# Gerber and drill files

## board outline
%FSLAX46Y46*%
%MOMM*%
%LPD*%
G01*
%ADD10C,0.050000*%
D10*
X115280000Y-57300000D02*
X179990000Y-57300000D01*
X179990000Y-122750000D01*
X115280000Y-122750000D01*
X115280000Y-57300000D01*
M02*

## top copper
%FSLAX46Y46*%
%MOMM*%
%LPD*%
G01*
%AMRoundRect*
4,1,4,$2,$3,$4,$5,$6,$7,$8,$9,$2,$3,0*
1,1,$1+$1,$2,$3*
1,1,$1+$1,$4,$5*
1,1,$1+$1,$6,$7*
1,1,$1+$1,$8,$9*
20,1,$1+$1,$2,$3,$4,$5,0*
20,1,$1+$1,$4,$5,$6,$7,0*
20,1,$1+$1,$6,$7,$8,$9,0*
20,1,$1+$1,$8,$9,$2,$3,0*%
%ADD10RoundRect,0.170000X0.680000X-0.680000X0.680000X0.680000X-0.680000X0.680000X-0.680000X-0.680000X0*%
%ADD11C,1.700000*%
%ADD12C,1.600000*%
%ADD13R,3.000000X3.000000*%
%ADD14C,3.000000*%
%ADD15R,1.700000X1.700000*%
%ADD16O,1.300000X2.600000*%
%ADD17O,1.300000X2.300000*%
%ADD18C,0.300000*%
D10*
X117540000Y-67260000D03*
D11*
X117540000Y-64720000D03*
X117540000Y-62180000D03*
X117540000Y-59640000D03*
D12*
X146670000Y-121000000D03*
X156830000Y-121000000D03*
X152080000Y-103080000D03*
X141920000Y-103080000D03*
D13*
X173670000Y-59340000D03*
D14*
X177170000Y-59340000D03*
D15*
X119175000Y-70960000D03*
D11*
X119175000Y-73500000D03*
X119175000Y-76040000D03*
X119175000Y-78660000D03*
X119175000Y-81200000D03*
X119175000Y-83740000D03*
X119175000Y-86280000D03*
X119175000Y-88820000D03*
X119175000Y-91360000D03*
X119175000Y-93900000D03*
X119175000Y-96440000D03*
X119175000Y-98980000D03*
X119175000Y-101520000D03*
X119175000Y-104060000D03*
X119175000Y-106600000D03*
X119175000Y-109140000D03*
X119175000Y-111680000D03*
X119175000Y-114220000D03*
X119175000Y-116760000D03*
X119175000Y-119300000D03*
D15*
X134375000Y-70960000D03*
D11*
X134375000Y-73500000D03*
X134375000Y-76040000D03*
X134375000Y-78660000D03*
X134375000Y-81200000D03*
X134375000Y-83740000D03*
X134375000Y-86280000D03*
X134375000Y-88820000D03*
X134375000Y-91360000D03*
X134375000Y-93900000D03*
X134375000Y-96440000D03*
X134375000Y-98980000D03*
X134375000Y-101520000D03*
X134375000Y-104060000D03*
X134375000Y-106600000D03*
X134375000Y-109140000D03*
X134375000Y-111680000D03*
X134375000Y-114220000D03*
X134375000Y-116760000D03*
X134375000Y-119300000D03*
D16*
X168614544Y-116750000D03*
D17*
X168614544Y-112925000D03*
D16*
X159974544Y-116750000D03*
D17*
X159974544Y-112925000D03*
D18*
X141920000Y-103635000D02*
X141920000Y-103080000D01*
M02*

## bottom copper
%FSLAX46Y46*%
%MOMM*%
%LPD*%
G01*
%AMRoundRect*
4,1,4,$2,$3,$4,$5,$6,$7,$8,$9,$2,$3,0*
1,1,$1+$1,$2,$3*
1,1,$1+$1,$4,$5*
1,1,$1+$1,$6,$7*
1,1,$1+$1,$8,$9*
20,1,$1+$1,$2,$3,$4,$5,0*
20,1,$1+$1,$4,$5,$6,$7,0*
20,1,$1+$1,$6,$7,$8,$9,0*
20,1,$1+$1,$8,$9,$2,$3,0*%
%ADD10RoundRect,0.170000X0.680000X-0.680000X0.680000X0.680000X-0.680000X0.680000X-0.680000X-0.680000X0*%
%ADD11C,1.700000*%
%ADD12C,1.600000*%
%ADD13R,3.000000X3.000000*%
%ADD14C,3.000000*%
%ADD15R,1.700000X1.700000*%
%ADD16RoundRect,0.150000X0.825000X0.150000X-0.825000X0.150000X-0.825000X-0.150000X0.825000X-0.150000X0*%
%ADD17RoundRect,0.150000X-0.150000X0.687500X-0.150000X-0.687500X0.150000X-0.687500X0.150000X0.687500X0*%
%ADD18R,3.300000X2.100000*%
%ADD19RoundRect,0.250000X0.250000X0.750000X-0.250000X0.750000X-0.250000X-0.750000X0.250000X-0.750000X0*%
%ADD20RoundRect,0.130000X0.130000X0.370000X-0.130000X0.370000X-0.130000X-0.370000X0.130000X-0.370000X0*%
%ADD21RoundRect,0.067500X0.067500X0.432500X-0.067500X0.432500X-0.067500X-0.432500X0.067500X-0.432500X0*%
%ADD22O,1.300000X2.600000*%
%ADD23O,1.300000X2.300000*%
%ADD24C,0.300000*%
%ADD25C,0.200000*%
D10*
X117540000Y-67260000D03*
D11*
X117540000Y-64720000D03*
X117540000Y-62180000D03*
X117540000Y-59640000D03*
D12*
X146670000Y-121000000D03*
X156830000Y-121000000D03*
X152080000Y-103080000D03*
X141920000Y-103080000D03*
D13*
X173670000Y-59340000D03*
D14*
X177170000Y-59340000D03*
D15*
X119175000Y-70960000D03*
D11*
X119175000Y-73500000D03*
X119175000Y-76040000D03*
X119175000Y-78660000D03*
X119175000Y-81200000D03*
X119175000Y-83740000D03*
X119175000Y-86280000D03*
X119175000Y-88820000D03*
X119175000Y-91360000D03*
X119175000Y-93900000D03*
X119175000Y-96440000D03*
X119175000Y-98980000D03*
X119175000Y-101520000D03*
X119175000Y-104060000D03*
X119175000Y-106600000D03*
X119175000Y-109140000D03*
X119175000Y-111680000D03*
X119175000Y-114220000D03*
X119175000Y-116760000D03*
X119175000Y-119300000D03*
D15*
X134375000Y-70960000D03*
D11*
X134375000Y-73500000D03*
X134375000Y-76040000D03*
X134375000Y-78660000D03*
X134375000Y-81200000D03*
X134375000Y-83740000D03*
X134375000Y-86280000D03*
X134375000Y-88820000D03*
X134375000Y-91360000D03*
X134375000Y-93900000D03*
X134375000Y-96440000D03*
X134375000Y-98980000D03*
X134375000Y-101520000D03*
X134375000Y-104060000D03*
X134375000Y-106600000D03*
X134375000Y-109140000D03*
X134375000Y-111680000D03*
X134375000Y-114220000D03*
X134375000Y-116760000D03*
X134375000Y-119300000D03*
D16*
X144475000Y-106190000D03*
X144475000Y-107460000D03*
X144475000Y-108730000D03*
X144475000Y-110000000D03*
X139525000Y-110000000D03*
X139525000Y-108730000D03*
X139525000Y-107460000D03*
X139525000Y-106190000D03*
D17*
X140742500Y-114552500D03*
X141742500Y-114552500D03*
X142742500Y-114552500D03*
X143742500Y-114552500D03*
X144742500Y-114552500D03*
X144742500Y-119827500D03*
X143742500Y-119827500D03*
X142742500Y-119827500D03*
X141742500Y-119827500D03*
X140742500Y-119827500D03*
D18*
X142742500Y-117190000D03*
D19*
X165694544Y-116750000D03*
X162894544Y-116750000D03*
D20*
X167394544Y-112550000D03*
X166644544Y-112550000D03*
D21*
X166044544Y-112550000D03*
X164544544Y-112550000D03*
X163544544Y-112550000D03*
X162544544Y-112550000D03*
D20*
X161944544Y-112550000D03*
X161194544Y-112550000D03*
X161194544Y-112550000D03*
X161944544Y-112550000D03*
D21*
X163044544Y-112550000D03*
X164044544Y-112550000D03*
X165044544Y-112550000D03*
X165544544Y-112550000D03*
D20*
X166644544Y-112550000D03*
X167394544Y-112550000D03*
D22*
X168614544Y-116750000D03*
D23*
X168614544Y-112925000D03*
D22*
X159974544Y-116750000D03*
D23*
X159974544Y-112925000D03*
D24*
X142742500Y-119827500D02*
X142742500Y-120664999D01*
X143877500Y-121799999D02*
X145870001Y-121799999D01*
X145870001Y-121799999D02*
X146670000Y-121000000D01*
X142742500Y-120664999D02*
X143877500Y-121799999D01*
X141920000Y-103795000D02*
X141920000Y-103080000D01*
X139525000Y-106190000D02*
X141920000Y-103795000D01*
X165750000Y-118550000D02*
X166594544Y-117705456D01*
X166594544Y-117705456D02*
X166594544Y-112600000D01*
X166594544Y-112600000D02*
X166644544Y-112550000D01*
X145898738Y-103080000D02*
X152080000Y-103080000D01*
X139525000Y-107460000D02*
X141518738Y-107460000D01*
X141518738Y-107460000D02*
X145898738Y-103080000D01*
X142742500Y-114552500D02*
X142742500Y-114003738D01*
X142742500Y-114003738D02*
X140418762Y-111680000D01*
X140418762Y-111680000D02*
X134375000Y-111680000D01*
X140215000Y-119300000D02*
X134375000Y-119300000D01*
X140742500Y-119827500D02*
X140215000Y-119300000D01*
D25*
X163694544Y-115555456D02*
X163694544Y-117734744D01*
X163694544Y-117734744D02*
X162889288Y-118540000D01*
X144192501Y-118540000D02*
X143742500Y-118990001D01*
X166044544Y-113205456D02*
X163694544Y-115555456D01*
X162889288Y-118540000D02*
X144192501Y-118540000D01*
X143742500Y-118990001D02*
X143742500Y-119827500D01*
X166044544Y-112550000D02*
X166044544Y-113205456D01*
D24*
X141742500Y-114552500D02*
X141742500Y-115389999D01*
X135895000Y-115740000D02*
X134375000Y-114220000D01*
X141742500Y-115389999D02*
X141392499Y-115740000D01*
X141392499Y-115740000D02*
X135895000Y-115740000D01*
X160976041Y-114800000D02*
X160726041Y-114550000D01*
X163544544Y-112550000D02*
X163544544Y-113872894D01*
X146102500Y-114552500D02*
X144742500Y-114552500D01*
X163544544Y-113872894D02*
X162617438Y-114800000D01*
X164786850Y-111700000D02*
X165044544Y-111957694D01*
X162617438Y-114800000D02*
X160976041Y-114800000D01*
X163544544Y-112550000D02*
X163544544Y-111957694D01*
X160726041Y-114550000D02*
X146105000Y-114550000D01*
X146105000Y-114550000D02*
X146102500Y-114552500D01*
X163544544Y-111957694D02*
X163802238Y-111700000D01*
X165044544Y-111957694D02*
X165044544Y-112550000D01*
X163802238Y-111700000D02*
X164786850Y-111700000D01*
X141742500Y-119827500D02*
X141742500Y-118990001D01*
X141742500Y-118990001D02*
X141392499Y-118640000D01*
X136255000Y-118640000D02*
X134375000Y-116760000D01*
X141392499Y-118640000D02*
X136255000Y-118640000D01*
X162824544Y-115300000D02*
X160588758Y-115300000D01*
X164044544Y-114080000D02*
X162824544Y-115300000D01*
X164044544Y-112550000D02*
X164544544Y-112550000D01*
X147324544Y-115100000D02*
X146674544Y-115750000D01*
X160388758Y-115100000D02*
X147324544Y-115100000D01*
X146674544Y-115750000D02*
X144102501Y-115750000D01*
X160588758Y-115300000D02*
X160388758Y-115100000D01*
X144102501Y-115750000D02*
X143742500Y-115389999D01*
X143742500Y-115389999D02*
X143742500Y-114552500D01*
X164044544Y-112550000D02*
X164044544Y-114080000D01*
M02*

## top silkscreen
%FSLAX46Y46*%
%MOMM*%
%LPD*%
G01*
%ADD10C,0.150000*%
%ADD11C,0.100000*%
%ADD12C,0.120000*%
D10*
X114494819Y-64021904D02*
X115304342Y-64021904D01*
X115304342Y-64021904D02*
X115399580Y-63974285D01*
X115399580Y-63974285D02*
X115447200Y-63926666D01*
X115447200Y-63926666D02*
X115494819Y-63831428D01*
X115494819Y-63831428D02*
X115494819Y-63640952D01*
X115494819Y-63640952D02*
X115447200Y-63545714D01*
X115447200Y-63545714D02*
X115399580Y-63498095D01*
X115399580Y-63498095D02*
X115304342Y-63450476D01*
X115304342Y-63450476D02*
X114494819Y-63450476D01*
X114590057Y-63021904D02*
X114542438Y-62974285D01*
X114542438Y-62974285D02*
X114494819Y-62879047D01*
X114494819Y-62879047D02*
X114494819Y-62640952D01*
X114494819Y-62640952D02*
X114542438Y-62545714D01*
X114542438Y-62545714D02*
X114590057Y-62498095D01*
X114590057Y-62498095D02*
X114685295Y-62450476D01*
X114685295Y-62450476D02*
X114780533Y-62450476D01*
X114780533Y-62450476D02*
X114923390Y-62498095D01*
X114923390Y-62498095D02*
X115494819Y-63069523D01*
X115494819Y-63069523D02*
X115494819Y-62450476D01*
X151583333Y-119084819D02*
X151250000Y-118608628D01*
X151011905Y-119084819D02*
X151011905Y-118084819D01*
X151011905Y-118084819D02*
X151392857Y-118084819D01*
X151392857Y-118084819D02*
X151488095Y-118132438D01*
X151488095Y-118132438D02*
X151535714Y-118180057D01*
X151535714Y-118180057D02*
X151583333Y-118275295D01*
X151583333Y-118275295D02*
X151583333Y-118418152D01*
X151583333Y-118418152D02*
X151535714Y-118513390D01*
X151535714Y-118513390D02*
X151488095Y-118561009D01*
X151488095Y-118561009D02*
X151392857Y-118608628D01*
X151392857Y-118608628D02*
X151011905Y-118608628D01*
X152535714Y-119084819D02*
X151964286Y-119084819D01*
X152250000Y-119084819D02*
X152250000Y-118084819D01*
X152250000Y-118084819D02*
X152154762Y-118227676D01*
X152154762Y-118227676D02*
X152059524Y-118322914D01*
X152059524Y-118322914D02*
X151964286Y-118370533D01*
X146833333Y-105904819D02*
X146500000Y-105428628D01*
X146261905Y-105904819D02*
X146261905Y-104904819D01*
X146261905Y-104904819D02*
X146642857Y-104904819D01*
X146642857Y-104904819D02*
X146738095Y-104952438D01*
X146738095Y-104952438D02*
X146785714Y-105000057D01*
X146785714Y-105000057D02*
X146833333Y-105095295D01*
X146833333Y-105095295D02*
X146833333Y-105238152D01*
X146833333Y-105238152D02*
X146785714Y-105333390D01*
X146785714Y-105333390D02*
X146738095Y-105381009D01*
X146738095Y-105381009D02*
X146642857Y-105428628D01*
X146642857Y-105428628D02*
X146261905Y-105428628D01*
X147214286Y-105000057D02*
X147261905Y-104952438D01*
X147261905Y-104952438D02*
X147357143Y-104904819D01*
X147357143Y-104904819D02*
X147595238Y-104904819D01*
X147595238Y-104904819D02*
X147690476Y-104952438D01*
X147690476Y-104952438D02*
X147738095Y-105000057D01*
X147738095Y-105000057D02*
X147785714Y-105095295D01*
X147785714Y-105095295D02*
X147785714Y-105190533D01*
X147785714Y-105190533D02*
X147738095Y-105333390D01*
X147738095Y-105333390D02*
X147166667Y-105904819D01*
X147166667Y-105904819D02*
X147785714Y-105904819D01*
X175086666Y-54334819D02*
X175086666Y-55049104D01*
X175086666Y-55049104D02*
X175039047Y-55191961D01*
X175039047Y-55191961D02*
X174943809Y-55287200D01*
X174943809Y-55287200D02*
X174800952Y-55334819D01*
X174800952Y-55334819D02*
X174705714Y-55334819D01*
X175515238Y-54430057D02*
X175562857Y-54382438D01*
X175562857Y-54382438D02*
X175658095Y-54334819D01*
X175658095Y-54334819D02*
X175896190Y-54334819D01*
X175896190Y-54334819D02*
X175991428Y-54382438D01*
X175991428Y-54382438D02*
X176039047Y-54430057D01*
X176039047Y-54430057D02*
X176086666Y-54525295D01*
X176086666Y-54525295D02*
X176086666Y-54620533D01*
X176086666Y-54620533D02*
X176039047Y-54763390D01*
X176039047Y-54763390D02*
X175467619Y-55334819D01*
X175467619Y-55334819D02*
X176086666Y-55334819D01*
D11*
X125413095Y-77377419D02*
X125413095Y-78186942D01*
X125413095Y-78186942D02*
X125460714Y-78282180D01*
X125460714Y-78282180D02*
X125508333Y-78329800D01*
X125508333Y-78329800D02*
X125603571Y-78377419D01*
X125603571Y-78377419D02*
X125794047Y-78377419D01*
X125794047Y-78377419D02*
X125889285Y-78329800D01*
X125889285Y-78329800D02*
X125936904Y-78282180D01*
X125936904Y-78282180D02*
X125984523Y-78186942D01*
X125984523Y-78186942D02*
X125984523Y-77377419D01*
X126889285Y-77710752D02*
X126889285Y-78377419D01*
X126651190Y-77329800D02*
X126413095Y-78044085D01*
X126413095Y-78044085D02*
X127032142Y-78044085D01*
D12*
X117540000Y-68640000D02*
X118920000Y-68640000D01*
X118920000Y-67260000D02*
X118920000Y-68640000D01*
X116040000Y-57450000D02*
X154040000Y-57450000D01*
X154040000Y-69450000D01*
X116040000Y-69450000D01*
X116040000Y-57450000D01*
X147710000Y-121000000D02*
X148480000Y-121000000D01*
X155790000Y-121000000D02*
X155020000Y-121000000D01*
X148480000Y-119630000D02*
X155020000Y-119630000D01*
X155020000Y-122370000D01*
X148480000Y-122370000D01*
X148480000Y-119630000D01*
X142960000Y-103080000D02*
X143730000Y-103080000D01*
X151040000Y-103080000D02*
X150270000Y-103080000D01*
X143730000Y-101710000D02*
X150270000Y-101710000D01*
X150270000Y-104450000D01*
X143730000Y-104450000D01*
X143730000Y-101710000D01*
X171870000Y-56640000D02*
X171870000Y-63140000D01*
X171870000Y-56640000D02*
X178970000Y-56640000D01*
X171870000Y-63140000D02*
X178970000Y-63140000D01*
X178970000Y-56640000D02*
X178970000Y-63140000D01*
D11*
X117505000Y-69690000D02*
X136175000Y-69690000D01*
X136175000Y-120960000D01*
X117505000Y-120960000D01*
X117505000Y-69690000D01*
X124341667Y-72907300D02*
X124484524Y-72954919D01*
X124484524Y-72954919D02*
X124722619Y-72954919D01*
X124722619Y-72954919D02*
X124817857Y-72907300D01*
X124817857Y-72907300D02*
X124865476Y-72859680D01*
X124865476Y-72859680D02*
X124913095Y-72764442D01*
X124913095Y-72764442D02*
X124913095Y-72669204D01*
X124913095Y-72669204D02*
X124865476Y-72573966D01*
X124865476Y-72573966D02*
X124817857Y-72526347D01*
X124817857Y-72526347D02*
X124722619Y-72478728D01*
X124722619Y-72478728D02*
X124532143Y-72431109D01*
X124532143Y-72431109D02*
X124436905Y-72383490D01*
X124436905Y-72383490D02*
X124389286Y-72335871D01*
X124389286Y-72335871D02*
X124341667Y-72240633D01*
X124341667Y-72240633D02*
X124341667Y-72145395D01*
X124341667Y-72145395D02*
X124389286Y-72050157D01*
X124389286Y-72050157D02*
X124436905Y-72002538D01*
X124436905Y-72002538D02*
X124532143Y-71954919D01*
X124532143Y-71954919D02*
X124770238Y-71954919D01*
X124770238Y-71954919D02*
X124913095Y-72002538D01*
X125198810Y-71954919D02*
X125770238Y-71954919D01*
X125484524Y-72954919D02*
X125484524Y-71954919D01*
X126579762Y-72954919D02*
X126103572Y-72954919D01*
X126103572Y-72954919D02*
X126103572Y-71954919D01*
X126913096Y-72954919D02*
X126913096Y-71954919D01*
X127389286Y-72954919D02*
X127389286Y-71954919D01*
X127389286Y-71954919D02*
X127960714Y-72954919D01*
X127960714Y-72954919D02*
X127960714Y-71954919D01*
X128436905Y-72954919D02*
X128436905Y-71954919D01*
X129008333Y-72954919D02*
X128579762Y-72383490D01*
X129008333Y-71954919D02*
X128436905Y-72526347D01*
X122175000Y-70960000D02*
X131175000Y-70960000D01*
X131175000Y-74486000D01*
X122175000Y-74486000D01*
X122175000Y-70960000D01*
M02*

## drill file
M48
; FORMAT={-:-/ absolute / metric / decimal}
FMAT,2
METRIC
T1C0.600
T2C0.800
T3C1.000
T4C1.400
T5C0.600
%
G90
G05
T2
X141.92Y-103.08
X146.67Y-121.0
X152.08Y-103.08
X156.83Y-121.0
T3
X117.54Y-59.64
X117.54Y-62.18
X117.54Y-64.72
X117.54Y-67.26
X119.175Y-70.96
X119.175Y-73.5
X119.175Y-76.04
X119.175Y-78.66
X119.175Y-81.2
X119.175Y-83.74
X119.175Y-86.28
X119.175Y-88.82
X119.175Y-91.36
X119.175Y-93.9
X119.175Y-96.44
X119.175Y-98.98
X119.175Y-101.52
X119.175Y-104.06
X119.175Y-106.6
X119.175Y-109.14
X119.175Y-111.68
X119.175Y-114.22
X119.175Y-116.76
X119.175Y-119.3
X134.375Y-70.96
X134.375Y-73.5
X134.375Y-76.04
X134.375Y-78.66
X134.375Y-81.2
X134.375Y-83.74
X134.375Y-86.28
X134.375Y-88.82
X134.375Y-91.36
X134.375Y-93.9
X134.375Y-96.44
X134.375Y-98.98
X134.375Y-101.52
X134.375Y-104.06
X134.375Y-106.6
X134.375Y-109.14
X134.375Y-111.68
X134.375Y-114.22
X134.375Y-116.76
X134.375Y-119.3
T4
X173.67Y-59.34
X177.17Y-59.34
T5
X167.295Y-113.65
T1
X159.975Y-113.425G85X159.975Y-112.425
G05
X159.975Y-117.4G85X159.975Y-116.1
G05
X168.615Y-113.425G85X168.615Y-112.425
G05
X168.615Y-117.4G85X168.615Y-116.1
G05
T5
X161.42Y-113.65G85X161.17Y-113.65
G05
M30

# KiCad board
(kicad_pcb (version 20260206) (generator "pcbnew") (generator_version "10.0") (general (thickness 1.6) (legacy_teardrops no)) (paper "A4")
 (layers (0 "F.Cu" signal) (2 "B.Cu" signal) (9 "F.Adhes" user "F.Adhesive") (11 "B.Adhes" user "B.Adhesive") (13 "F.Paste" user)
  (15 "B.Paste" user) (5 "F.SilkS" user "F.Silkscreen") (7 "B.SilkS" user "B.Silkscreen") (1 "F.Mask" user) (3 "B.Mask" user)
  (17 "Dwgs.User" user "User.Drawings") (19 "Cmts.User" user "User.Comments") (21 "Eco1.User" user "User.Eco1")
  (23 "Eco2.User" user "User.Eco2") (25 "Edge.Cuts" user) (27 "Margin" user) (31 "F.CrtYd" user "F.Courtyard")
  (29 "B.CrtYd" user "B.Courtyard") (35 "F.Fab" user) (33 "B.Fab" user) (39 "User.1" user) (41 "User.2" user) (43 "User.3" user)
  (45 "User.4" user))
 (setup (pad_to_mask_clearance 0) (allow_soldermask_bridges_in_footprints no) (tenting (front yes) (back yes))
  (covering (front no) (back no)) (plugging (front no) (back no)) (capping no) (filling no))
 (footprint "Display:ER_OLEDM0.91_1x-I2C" (layer "F.Cu") (at 117.54 67.26 90)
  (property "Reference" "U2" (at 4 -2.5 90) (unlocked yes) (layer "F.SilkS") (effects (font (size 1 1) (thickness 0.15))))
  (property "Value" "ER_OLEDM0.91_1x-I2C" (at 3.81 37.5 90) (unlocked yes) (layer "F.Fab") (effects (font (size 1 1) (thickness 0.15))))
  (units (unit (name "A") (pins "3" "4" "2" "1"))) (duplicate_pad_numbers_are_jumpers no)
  (fp_line (start -1.38 0) (end -1.38 1.38) (stroke (width 0.12) (type solid)) (layer "F.SilkS"))
  (fp_line (start 0 1.38) (end -1.38 1.38) (stroke (width 0.12) (type solid)) (layer "F.SilkS"))
  (fp_rect (start -2.19 -1.5) (end 9.81 36.5) (stroke (width 0.12) (type solid)) (fill no) (layer "F.SilkS"))
  (pad "1" thru_hole roundrect (at 0 0 90) (size 1.7 1.7) (drill 1) (layers "*.Cu" "*.Mask") (remove_unused_layers no)
   (roundrect_rratio 0.1) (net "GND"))
  (pad "2" thru_hole circle (at 2.54 0 90) (size 1.7 1.7) (drill 1) (layers "*.Cu" "*.Mask") (remove_unused_layers no) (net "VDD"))
  (pad "3" thru_hole circle (at 5.08 0 90) (size 1.7 1.7) (drill 1) (layers "*.Cu" "*.Mask") (remove_unused_layers no) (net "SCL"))
  (pad "4" thru_hole circle (at 7.62 0 90) (size 1.7 1.7) (drill 1) (layers "*.Cu" "*.Mask") (remove_unused_layers no) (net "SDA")))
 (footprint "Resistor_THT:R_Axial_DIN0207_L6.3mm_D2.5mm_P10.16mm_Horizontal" (layer "F.Cu") (at 146.67 121)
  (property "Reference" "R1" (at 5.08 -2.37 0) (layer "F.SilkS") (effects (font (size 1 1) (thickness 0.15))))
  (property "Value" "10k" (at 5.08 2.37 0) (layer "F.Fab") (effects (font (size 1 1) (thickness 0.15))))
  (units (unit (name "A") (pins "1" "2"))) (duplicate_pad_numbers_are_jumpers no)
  (fp_line (start 1.04 0) (end 1.81 0) (stroke (width 0.12) (type solid)) (layer "F.SilkS"))
  (fp_line (start 9.12 0) (end 8.35 0) (stroke (width 0.12) (type solid)) (layer "F.SilkS"))
  (fp_rect (start 1.81 -1.37) (end 8.35 1.37) (stroke (width 0.12) (type solid)) (fill no) (layer "F.SilkS"))
  (pad "1" thru_hole circle (at 0 0) (size 1.6 1.6) (drill 0.8) (layers "*.Cu" "*.Mask") (remove_unused_layers no) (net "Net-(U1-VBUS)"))
  (pad "2" thru_hole circle (at 10.16 0) (size 1.6 1.6) (drill 0.8) (layers "*.Cu" "*.Mask") (remove_unused_layers no) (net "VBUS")))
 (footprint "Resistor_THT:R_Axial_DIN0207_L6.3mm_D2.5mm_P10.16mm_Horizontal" (layer "F.Cu") (at 152.08 103.08 180)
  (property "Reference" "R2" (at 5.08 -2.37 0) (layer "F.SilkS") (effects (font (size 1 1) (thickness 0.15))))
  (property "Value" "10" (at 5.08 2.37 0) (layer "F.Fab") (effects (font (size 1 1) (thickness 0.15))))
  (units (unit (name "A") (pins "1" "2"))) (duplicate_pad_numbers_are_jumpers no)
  (fp_line (start 9.12 0) (end 8.35 0) (stroke (width 0.12) (type solid)) (layer "F.SilkS"))
  (fp_line (start 1.04 0) (end 1.81 0) (stroke (width 0.12) (type solid)) (layer "F.SilkS"))
  (fp_rect (start 1.81 -1.37) (end 8.35 1.37) (stroke (width 0.12) (type solid)) (fill no) (layer "F.SilkS"))
  (pad "1" thru_hole circle (at 0 0 180) (size 1.6 1.6) (drill 0.8) (layers "*.Cu" "*.Mask") (remove_unused_layers no) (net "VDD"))
  (pad "2" thru_hole circle (at 10.16 0 180) (size 1.6 1.6) (drill 0.8) (layers "*.Cu" "*.Mask") (remove_unused_layers no) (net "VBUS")))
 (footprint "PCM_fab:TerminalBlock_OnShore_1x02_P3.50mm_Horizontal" (layer "F.Cu") (at 173.67 59.34)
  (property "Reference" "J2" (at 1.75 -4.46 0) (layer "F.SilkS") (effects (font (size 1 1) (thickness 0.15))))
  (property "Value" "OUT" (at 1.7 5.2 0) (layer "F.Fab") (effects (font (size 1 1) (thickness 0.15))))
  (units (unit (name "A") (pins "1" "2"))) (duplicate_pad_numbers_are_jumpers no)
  (fp_line (start -1.8 -2.7) (end -1.8 3.8) (stroke (width 0.12) (type solid)) (layer "F.SilkS"))
  (fp_line (start -1.8 -2.7) (end 5.3 -2.7) (stroke (width 0.12) (type solid)) (layer "F.SilkS"))
  (fp_line (start -1.8 3.8) (end 5.3 3.8) (stroke (width 0.12) (type solid)) (layer "F.SilkS"))
  (fp_line (start 5.3 -2.7) (end 5.3 3.8) (stroke (width 0.12) (type solid)) (layer "F.SilkS"))
  (pad "1" thru_hole rect (at 0 0) (size 3 3) (drill 1.4) (layers "*.Cu" "*.Mask") (remove_unused_layers no) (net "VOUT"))
  (pad "2" thru_hole circle (at 3.5 0) (size 3 3) (drill 1.4) (layers "*.Cu" "*.Mask") (remove_unused_layers no) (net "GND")))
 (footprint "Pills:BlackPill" (layer "F.Cu") (at 119.175 65.96)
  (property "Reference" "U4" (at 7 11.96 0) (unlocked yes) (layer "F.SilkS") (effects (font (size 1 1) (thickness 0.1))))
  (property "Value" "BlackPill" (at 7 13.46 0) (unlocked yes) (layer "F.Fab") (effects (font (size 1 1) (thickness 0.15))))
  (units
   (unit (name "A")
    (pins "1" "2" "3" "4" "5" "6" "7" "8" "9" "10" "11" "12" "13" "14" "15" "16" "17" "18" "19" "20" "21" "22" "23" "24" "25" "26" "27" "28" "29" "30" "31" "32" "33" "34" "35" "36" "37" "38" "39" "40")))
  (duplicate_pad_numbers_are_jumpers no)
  (fp_rect (start -1.67 3.73) (end 17 55) (stroke (width 0.1) (type default)) (fill no) (layer "F.SilkS"))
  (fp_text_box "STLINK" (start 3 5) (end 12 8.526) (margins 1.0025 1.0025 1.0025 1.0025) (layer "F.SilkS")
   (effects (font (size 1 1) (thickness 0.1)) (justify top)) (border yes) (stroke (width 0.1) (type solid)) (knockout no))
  (pad "1" thru_hole rect (at 0 5) (size 1.7 1.7) (drill 1) (layers "*.Cu" "*.Mask") (remove_unused_layers no)
   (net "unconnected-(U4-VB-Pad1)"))
  (pad "2" thru_hole circle (at 0 7.54) (size 1.7 1.7) (drill 1) (layers "*.Cu" "*.Mask") (remove_unused_layers no)
   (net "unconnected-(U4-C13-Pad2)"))
  (pad "3" thru_hole circle (at 0 10.08) (size 1.7 1.7) (drill 1) (layers "*.Cu" "*.Mask") (remove_unused_layers no)
   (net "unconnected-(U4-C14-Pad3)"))
  (pad "4" thru_hole circle (at 0 12.7) (size 1.7 1.7) (drill 1) (layers "*.Cu" "*.Mask") (remove_unused_layers no)
   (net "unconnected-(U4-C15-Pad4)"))
  (pad "5" thru_hole circle (at 0 15.24) (size 1.7 1.7) (drill 1) (layers "*.Cu" "*.Mask") (remove_unused_layers no)
   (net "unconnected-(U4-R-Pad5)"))
  (pad "6" thru_hole circle (at 0 17.78) (size 1.7 1.7) (drill 1) (layers "*.Cu" "*.Mask") (remove_unused_layers no)
   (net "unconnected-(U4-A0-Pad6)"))
  (pad "7" thru_hole circle (at 0 20.32) (size 1.7 1.7) (drill 1) (layers "*.Cu" "*.Mask") (remove_unused_layers no)
   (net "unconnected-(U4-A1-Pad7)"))
  (pad "8" thru_hole circle (at 0 22.86) (size 1.7 1.7) (drill 1) (layers "*.Cu" "*.Mask") (remove_unused_layers no)
   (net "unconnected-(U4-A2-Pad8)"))
  (pad "9" thru_hole circle (at 0 25.4) (size 1.7 1.7) (drill 1) (layers "*.Cu" "*.Mask") (remove_unused_layers no)
   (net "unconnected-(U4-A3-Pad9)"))
  (pad "10" thru_hole circle (at 0 27.94) (size 1.7 1.7) (drill 1) (layers "*.Cu" "*.Mask") (remove_unused_layers no)
   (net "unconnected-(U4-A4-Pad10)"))
  (pad "11" thru_hole circle (at 0 30.48) (size 1.7 1.7) (drill 1) (layers "*.Cu" "*.Mask") (remove_unused_layers no)
   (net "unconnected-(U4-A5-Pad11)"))
  (pad "12" thru_hole circle (at 0 33.02) (size 1.7 1.7) (drill 1) (layers "*.Cu" "*.Mask") (remove_unused_layers no)
   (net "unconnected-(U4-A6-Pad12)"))
  (pad "13" thru_hole circle (at 0 35.56) (size 1.7 1.7) (drill 1) (layers "*.Cu" "*.Mask") (remove_unused_layers no)
   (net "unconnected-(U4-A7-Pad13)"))
  (pad "14" thru_hole circle (at 0 38.1) (size 1.7 1.7) (drill 1) (layers "*.Cu" "*.Mask") (remove_unused_layers no)
   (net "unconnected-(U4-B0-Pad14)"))
  (pad "15" thru_hole circle (at 0 40.64) (size 1.7 1.7) (drill 1) (layers "*.Cu" "*.Mask") (remove_unused_layers no)
   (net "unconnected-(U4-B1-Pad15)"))
  (pad "16" thru_hole circle (at 0 43.18) (size 1.7 1.7) (drill 1) (layers "*.Cu" "*.Mask") (remove_unused_layers no)
   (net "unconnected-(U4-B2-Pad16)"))
  (pad "17" thru_hole circle (at 0 45.72) (size 1.7 1.7) (drill 1) (layers "*.Cu" "*.Mask") (remove_unused_layers no)
   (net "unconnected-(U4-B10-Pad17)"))
  (pad "18" thru_hole circle (at 0 48.26) (size 1.7 1.7) (drill 1) (layers "*.Cu" "*.Mask") (remove_unused_layers no)
   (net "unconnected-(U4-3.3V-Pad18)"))
  (pad "19" thru_hole circle (at 0 50.8) (size 1.7 1.7) (drill 1) (layers "*.Cu" "*.Mask") (remove_unused_layers no)
   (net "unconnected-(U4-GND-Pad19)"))
  (pad "20" thru_hole circle (at 0 53.34) (size 1.7 1.7) (drill 1) (layers "*.Cu" "*.Mask") (remove_unused_layers no)
   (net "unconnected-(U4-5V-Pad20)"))
  (pad "21" thru_hole rect (at 15.2 5) (size 1.7 1.7) (drill 1) (layers "*.Cu" "*.Mask") (remove_unused_layers no)
   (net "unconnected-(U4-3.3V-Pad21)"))
  (pad "22" thru_hole circle (at 15.2 7.54) (size 1.7 1.7) (drill 1) (layers "*.Cu" "*.Mask") (remove_unused_layers no)
   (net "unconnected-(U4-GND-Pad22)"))
  (pad "23" thru_hole circle (at 15.2 10.08) (size 1.7 1.7) (drill 1) (layers "*.Cu" "*.Mask") (remove_unused_layers no)
   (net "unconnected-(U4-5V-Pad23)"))
  (pad "24" thru_hole circle (at 15.2 12.7) (size 1.7 1.7) (drill 1) (layers "*.Cu" "*.Mask") (remove_unused_layers no)
   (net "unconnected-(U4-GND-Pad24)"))
  (pad "25" thru_hole circle (at 15.2 15.24) (size 1.7 1.7) (drill 1) (layers "*.Cu" "*.Mask") (remove_unused_layers no)
   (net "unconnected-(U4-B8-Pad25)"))
  (pad "26" thru_hole circle (at 15.2 17.78) (size 1.7 1.7) (drill 1) (layers "*.Cu" "*.Mask") (remove_unused_layers no) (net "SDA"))
  (pad "27" thru_hole circle (at 15.2 20.32) (size 1.7 1.7) (drill 1) (layers "*.Cu" "*.Mask") (remove_unused_layers no) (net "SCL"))
  (pad "28" thru_hole circle (at 15.2 22.86) (size 1.7 1.7) (drill 1) (layers "*.Cu" "*.Mask") (remove_unused_layers no)
   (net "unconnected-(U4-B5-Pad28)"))
  (pad "29" thru_hole circle (at 15.2 25.4) (size 1.7 1.7) (drill 1) (layers "*.Cu" "*.Mask") (remove_unused_layers no)
   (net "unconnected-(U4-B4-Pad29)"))
  (pad "30" thru_hole circle (at 15.2 27.94) (size 1.7 1.7) (drill 1) (layers "*.Cu" "*.Mask") (remove_unused_layers no)
   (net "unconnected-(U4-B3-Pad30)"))
  (pad "31" thru_hole circle (at 15.2 30.48) (size 1.7 1.7) (drill 1) (layers "*.Cu" "*.Mask") (remove_unused_layers no)
   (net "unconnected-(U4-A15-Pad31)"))
  (pad "32" thru_hole circle (at 15.2 33.02) (size 1.7 1.7) (drill 1) (layers "*.Cu" "*.Mask") (remove_unused_layers no)
   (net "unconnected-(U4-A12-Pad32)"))
  (pad "33" thru_hole circle (at 15.2 35.56) (size 1.7 1.7) (drill 1) (layers "*.Cu" "*.Mask") (remove_unused_layers no)
   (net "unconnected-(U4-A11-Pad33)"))
  (pad "34" thru_hole circle (at 15.2 38.1) (size 1.7 1.7) (drill 1) (layers "*.Cu" "*.Mask") (remove_unused_layers no)
   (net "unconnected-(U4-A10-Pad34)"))
  (pad "35" thru_hole circle (at 15.2 40.64) (size 1.7 1.7) (drill 1) (layers "*.Cu" "*.Mask") (remove_unused_layers no)
   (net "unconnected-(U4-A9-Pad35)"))
  (pad "36" thru_hole circle (at 15.2 43.18) (size 1.7 1.7) (drill 1) (layers "*.Cu" "*.Mask") (remove_unused_layers no)
   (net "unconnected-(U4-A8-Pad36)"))
  (pad "37" thru_hole circle (at 15.2 45.72) (size 1.7 1.7) (drill 1) (layers "*.Cu" "*.Mask") (remove_unused_layers no) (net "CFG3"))
  (pad "38" thru_hole circle (at 15.2 48.26) (size 1.7 1.7) (drill 1) (layers "*.Cu" "*.Mask") (remove_unused_layers no) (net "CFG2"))
  (pad "39" thru_hole circle (at 15.2 50.8) (size 1.7 1.7) (drill 1) (layers "*.Cu" "*.Mask") (remove_unused_layers no) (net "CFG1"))
  (pad "40" thru_hole circle (at 15.2 53.34) (size 1.7 1.7) (drill 1) (layers "*.Cu" "*.Mask") (remove_unused_layers no) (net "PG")))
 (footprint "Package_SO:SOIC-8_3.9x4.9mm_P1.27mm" (layer "B.Cu") (at 142 108.095 180)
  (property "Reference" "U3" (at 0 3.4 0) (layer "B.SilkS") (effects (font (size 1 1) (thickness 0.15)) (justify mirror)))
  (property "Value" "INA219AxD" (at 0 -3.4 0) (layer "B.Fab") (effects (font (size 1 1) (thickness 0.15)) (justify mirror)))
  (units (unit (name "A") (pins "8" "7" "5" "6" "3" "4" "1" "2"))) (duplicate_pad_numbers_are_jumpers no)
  (pad "1" smd roundrect (at -2.475 1.905 180) (size 1.95 0.6) (layers "B.Cu" "B.Mask" "B.Paste") (roundrect_rratio 0.25) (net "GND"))
  (pad "2" smd roundrect (at -2.475 0.635 180) (size 1.95 0.6) (layers "B.Cu" "B.Mask" "B.Paste") (roundrect_rratio 0.25) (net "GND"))
  (pad "3" smd roundrect (at -2.475 -0.635 180) (size 1.95 0.6) (layers "B.Cu" "B.Mask" "B.Paste") (roundrect_rratio 0.25) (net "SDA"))
  (pad "4" smd roundrect (at -2.475 -1.905 180) (size 1.95 0.6) (layers "B.Cu" "B.Mask" "B.Paste") (roundrect_rratio 0.25) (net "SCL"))
  (pad "5" smd roundrect (at 2.475 -1.905 180) (size 1.95 0.6) (layers "B.Cu" "B.Mask" "B.Paste") (roundrect_rratio 0.25) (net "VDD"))
  (pad "6" smd roundrect (at 2.475 -0.635 180) (size 1.95 0.6) (layers "B.Cu" "B.Mask" "B.Paste") (roundrect_rratio 0.25) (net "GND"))
  (pad "7" smd roundrect (at 2.475 0.635 180) (size 1.95 0.6) (layers "B.Cu" "B.Mask" "B.Paste") (roundrect_rratio 0.25) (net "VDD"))
  (pad "8" smd roundrect (at 2.475 1.905 180) (size 1.95 0.6) (layers "B.Cu" "B.Mask" "B.Paste") (roundrect_rratio 0.25) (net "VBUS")))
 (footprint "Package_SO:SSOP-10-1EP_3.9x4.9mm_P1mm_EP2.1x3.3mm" (layer "B.Cu") (at 142.7425 117.19 -90)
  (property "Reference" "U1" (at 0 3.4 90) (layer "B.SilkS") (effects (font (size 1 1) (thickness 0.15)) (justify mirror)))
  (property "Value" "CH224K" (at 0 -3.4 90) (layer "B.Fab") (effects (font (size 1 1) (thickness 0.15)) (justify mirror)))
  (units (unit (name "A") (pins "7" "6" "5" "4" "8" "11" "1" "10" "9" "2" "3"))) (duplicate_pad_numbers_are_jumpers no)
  (pad "" smd roundrect (at 0 0 270) (size 1.69 2.66) (layers "B.Paste") (roundrect_rratio 0.147929))
  (pad "1" smd roundrect (at -2.6375 2 270) (size 1.675 0.6) (layers "B.Cu" "B.Mask" "B.Paste") (roundrect_rratio 0.25) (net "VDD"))
  (pad "2" smd roundrect (at -2.6375 1 270) (size 1.675 0.6) (layers "B.Cu" "B.Mask" "B.Paste") (roundrect_rratio 0.25) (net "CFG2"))
  (pad "3" smd roundrect (at -2.6375 0 270) (size 1.675 0.6) (layers "B.Cu" "B.Mask" "B.Paste") (roundrect_rratio 0.25) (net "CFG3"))
  (pad "4" smd roundrect (at -2.6375 -1 270) (size 1.675 0.6) (layers "B.Cu" "B.Mask" "B.Paste") (roundrect_rratio 0.25) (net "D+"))
  (pad "5" smd roundrect (at -2.6375 -2 270) (size 1.675 0.6) (layers "B.Cu" "B.Mask" "B.Paste") (roundrect_rratio 0.25) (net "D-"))
  (pad "6" smd roundrect (at 2.6375 -2 270) (size 1.675 0.6) (layers "B.Cu" "B.Mask" "B.Paste") (roundrect_rratio 0.25) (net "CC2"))
  (pad "7" smd roundrect (at 2.6375 -1 270) (size 1.675 0.6) (layers "B.Cu" "B.Mask" "B.Paste") (roundrect_rratio 0.25) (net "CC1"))
  (pad "8" smd roundrect (at 2.6375 0 270) (size 1.675 0.6) (layers "B.Cu" "B.Mask" "B.Paste") (roundrect_rratio 0.25) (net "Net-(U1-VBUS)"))
  (pad "9" smd roundrect (at 2.6375 1 270) (size 1.675 0.6) (layers "B.Cu" "B.Mask" "B.Paste") (roundrect_rratio 0.25) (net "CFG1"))
  (pad "10" smd roundrect (at 2.6375 2 270) (size 1.675 0.6) (layers "B.Cu" "B.Mask" "B.Paste") (roundrect_rratio 0.25) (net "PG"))
  (pad "11" smd rect (at 0 0 270) (size 2.1 3.3) (layers "B.Cu" "B.Mask") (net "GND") (zone_connect 2)))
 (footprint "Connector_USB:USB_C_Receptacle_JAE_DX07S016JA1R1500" (layer "B.Cu") (at 164.294544 115.6 180)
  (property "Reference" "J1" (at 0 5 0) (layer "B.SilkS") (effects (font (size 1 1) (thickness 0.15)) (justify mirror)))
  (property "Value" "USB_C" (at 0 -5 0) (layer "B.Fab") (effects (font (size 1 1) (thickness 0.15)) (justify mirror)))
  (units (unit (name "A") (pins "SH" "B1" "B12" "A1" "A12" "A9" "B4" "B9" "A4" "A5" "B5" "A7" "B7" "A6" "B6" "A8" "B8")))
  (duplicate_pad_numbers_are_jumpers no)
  (pad "" np_thru_hole circle (at -3 1.95 180) (size 0.6 0.6) (drill 0.6) (layers "*.Cu" "*.Mask"))
  (pad "" smd roundrect (at -1.4 -1.15 180) (size 1 2) (layers "B.Cu" "B.Mask" "B.Paste") (roundrect_rratio 0.25))
  (pad "" smd roundrect (at 1.4 -1.15 180) (size 1 2) (layers "B.Cu" "B.Mask" "B.Paste") (roundrect_rratio 0.25))
  (pad "" np_thru_hole oval (at 3 1.95 180) (size 0.85 0.6) (drill oval 0.85 0.6) (layers "*.Cu" "*.Mask"))
  (pad "A1" smd roundrect (at -3.1 3.05 180) (size 0.52 1) (layers "B.Cu" "B.Mask" "B.Paste") (roundrect_rratio 0.25) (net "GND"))
  (pad "A4" smd roundrect (at -2.35 3.05 180) (size 0.52 1) (layers "B.Cu" "B.Mask" "B.Paste") (roundrect_rratio 0.25) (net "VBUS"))
  (pad "A5" smd roundrect (at -1.75 3.05 180) (size 0.27 1) (layers "B.Cu" "B.Mask" "B.Paste") (roundrect_rratio 0.25) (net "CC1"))
  (pad "A6" smd roundrect (at -0.25 3.05 180) (size 0.27 1) (layers "B.Cu" "B.Mask" "B.Paste") (roundrect_rratio 0.25) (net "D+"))
  (pad "A7" smd roundrect (at 0.75 3.05 180) (size 0.27 1) (layers "B.Cu" "B.Mask" "B.Paste") (roundrect_rratio 0.25) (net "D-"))
  (pad "A8" smd roundrect (at 1.75 3.05 180) (size 0.27 1) (layers "B.Cu" "B.Mask" "B.Paste") (roundrect_rratio 0.25)
   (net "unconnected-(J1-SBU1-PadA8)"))
  (pad "A9" smd roundrect (at 2.35 3.05 180) (size 0.52 1) (layers "B.Cu" "B.Mask" "B.Paste") (roundrect_rratio 0.25) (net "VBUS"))
  (pad "A12" smd roundrect (at 3.1 3.05 180) (size 0.52 1) (layers "B.Cu" "B.Mask" "B.Paste") (roundrect_rratio 0.25) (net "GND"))
  (pad "B1" smd roundrect (at 3.1 3.05 180) (size 0.52 1) (layers "B.Cu" "B.Mask" "B.Paste") (roundrect_rratio 0.25) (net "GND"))
  (pad "B4" smd roundrect (at 2.35 3.05 180) (size 0.52 1) (layers "B.Cu" "B.Mask" "B.Paste") (roundrect_rratio 0.25) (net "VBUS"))
  (pad "B5" smd roundrect (at 1.25 3.05 180) (size 0.27 1) (layers "B.Cu" "B.Mask" "B.Paste") (roundrect_rratio 0.25) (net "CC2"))
  (pad "B6" smd roundrect (at 0.25 3.05 180) (size 0.27 1) (layers "B.Cu" "B.Mask" "B.Paste") (roundrect_rratio 0.25) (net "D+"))
  (pad "B7" smd roundrect (at -0.75 3.05 180) (size 0.27 1) (layers "B.Cu" "B.Mask" "B.Paste") (roundrect_rratio 0.25) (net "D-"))
  (pad "B8" smd roundrect (at -1.25 3.05 180) (size 0.27 1) (layers "B.Cu" "B.Mask" "B.Paste") (roundrect_rratio 0.25)
   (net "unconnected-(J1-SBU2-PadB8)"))
  (pad "B9" smd roundrect (at -2.35 3.05 180) (size 0.52 1) (layers "B.Cu" "B.Mask" "B.Paste") (roundrect_rratio 0.25) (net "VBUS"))
  (pad "B12" smd roundrect (at -3.1 3.05 180) (size 0.52 1) (layers "B.Cu" "B.Mask" "B.Paste") (roundrect_rratio 0.25) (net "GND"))
  (pad "SH" thru_hole oval (at -4.32 -1.15 180) (size 1.3 2.6) (drill oval 0.6 1.9) (layers "*.Cu" "*.Mask") (remove_unused_layers no)
   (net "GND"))
  (pad "SH" thru_hole oval (at -4.32 2.675 180) (size 1.3 2.3) (drill oval 0.6 1.6) (layers "*.Cu" "*.Mask") (remove_unused_layers no)
   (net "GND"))
  (pad "SH" thru_hole oval (at 4.32 -1.15 180) (size 1.3 2.6) (drill oval 0.6 1.9) (layers "*.Cu" "*.Mask") (remove_unused_layers no)
   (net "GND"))
  (pad "SH" thru_hole oval (at 4.32 2.675 180) (size 1.3 2.3) (drill oval 0.6 1.6) (layers "*.Cu" "*.Mask") (remove_unused_layers no)
   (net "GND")))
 (gr_rect (start 115.28 57.3) (end 179.99 122.75) (stroke (width 0.05) (type default)) (fill no) (layer "Edge.Cuts"))
 (segment (start 142.7425 119.8275) (end 142.7425 120.664999) (width 0.3) (layer "B.Cu") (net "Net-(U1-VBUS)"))
 (segment (start 143.8775 121.799999) (end 145.870001 121.799999) (width 0.3) (layer "B.Cu") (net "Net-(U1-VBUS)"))
 (segment (start 145.870001 121.799999) (end 146.67 121) (width 0.3) (layer "B.Cu") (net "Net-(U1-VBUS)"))
 (segment (start 142.7425 120.664999) (end 143.8775 121.799999) (width 0.3) (layer "B.Cu") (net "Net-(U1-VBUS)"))
 (segment (start 141.92 103.635) (end 141.92 103.08) (width 0.3) (layer "F.Cu") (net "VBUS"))
 (segment (start 141.92 103.795) (end 141.92 103.08) (width 0.3) (layer "B.Cu") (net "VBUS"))
 (segment (start 139.525 106.19) (end 141.92 103.795) (width 0.3) (layer "B.Cu") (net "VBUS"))
 (segment (start 165.75 118.55) (end 166.594544 117.705456) (width 0.3) (layer "B.Cu") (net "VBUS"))
 (segment (start 166.594544 117.705456) (end 166.594544 112.6) (width 0.3) (layer "B.Cu") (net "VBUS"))
 (segment (start 166.594544 112.6) (end 166.644544 112.55) (width 0.3) (layer "B.Cu") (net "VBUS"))
 (segment (start 145.898738 103.08) (end 152.08 103.08) (width 0.3) (layer "B.Cu") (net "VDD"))
 (segment (start 139.525 107.46) (end 141.518738 107.46) (width 0.3) (layer "B.Cu") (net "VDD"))
 (segment (start 141.518738 107.46) (end 145.898738 103.08) (width 0.3) (layer "B.Cu") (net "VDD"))
 (segment (start 142.7425 114.5525) (end 142.7425 114.003738) (width 0.3) (layer "B.Cu") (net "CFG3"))
 (segment (start 142.7425 114.003738) (end 140.418762 111.68) (width 0.3) (layer "B.Cu") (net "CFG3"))
 (segment (start 140.418762 111.68) (end 134.375 111.68) (width 0.3) (layer "B.Cu") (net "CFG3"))
 (segment (start 140.215 119.3) (end 134.375 119.3) (width 0.3) (layer "B.Cu") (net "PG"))
 (segment (start 140.7425 119.8275) (end 140.215 119.3) (width 0.3) (layer "B.Cu") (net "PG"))
 (segment (start 163.694544 115.555456) (end 163.694544 117.734744) (width 0.2) (layer "B.Cu") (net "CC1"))
 (segment (start 163.694544 117.734744) (end 162.889288 118.54) (width 0.2) (layer "B.Cu") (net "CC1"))
 (segment (start 144.192501 118.54) (end 143.7425 118.990001) (width 0.2) (layer "B.Cu") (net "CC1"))
 (segment (start 166.044544 113.205456) (end 163.694544 115.555456) (width 0.2) (layer "B.Cu") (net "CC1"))
 (segment (start 162.889288 118.54) (end 144.192501 118.54) (width 0.2) (layer "B.Cu") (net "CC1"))
 (segment (start 143.7425 118.990001) (end 143.7425 119.8275) (width 0.2) (layer "B.Cu") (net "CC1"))
 (segment (start 166.044544 112.55) (end 166.044544 113.205456) (width 0.2) (layer "B.Cu") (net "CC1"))
 (segment (start 141.7425 114.5525) (end 141.7425 115.389999) (width 0.3) (layer "B.Cu") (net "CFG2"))
 (segment (start 135.895 115.74) (end 134.375 114.22) (width 0.3) (layer "B.Cu") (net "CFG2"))
 (segment (start 141.7425 115.389999) (end 141.392499 115.74) (width 0.3) (layer "B.Cu") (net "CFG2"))
 (segment (start 141.392499 115.74) (end 135.895 115.74) (width 0.3) (layer "B.Cu") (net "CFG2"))
 (segment (start 160.976041 114.8) (end 160.726041 114.55) (width 0.3) (layer "B.Cu") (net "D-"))
 (segment (start 163.544544 112.55) (end 163.544544 113.872894) (width 0.3) (layer "B.Cu") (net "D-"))
 (segment (start 146.1025 114.5525) (end 144.7425 114.5525) (width 0.3) (layer "B.Cu") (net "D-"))
 (segment (start 163.544544 113.872894) (end 162.617438 114.8) (width 0.3) (layer "B.Cu") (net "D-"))
 (segment (start 164.78685 111.7) (end 165.044544 111.957694) (width 0.3) (layer "B.Cu") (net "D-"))
 (segment (start 162.617438 114.8) (end 160.976041 114.8) (width 0.3) (layer "B.Cu") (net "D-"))
 (segment (start 163.544544 112.55) (end 163.544544 111.957694) (width 0.3) (layer "B.Cu") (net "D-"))
 (segment (start 160.726041 114.55) (end 146.105 114.55) (width 0.3) (layer "B.Cu") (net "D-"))
 (segment (start 146.105 114.55) (end 146.1025 114.5525) (width 0.3) (layer "B.Cu") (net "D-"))
 (segment (start 163.544544 111.957694) (end 163.802238 111.7) (width 0.3) (layer "B.Cu") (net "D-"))
 (segment (start 165.044544 111.957694) (end 165.044544 112.55) (width 0.3) (layer "B.Cu") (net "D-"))
 (segment (start 163.802238 111.7) (end 164.78685 111.7) (width 0.3) (layer "B.Cu") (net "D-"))
 (segment (start 141.7425 119.8275) (end 141.7425 118.990001) (width 0.3) (layer "B.Cu") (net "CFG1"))
 (segment (start 141.7425 118.990001) (end 141.392499 118.64) (width 0.3) (layer "B.Cu") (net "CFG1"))
 (segment (start 136.255 118.64) (end 134.375 116.76) (width 0.3) (layer "B.Cu") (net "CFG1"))
 (segment (start 141.392499 118.64) (end 136.255 118.64) (width 0.3) (layer "B.Cu") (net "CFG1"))
 (segment (start 162.824544 115.3) (end 160.588758 115.3) (width 0.3) (layer "B.Cu") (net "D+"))
 (segment (start 164.044544 114.08) (end 162.824544 115.3) (width 0.3) (layer "B.Cu") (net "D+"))
 (segment (start 164.044544 112.55) (end 164.544544 112.55) (width 0.3) (layer "B.Cu") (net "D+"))
 (segment (start 147.324544 115.1) (end 146.674544 115.75) (width 0.3) (layer "B.Cu") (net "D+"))
 (segment (start 160.388758 115.1) (end 147.324544 115.1) (width 0.3) (layer "B.Cu") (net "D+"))
 (segment (start 146.674544 115.75) (end 144.102501 115.75) (width 0.3) (layer "B.Cu") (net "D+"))
 (segment (start 160.588758 115.3) (end 160.388758 115.1) (width 0.3) (layer "B.Cu") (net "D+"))
 (segment (start 144.102501 115.75) (end 143.7425 115.389999) (width 0.3) (layer "B.Cu") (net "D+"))
 (segment (start 143.7425 115.389999) (end 143.7425 114.5525) (width 0.3) (layer "B.Cu") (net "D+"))
 (segment (start 164.044544 112.55) (end 164.044544 114.08) (width 0.3) (layer "B.Cu") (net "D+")))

